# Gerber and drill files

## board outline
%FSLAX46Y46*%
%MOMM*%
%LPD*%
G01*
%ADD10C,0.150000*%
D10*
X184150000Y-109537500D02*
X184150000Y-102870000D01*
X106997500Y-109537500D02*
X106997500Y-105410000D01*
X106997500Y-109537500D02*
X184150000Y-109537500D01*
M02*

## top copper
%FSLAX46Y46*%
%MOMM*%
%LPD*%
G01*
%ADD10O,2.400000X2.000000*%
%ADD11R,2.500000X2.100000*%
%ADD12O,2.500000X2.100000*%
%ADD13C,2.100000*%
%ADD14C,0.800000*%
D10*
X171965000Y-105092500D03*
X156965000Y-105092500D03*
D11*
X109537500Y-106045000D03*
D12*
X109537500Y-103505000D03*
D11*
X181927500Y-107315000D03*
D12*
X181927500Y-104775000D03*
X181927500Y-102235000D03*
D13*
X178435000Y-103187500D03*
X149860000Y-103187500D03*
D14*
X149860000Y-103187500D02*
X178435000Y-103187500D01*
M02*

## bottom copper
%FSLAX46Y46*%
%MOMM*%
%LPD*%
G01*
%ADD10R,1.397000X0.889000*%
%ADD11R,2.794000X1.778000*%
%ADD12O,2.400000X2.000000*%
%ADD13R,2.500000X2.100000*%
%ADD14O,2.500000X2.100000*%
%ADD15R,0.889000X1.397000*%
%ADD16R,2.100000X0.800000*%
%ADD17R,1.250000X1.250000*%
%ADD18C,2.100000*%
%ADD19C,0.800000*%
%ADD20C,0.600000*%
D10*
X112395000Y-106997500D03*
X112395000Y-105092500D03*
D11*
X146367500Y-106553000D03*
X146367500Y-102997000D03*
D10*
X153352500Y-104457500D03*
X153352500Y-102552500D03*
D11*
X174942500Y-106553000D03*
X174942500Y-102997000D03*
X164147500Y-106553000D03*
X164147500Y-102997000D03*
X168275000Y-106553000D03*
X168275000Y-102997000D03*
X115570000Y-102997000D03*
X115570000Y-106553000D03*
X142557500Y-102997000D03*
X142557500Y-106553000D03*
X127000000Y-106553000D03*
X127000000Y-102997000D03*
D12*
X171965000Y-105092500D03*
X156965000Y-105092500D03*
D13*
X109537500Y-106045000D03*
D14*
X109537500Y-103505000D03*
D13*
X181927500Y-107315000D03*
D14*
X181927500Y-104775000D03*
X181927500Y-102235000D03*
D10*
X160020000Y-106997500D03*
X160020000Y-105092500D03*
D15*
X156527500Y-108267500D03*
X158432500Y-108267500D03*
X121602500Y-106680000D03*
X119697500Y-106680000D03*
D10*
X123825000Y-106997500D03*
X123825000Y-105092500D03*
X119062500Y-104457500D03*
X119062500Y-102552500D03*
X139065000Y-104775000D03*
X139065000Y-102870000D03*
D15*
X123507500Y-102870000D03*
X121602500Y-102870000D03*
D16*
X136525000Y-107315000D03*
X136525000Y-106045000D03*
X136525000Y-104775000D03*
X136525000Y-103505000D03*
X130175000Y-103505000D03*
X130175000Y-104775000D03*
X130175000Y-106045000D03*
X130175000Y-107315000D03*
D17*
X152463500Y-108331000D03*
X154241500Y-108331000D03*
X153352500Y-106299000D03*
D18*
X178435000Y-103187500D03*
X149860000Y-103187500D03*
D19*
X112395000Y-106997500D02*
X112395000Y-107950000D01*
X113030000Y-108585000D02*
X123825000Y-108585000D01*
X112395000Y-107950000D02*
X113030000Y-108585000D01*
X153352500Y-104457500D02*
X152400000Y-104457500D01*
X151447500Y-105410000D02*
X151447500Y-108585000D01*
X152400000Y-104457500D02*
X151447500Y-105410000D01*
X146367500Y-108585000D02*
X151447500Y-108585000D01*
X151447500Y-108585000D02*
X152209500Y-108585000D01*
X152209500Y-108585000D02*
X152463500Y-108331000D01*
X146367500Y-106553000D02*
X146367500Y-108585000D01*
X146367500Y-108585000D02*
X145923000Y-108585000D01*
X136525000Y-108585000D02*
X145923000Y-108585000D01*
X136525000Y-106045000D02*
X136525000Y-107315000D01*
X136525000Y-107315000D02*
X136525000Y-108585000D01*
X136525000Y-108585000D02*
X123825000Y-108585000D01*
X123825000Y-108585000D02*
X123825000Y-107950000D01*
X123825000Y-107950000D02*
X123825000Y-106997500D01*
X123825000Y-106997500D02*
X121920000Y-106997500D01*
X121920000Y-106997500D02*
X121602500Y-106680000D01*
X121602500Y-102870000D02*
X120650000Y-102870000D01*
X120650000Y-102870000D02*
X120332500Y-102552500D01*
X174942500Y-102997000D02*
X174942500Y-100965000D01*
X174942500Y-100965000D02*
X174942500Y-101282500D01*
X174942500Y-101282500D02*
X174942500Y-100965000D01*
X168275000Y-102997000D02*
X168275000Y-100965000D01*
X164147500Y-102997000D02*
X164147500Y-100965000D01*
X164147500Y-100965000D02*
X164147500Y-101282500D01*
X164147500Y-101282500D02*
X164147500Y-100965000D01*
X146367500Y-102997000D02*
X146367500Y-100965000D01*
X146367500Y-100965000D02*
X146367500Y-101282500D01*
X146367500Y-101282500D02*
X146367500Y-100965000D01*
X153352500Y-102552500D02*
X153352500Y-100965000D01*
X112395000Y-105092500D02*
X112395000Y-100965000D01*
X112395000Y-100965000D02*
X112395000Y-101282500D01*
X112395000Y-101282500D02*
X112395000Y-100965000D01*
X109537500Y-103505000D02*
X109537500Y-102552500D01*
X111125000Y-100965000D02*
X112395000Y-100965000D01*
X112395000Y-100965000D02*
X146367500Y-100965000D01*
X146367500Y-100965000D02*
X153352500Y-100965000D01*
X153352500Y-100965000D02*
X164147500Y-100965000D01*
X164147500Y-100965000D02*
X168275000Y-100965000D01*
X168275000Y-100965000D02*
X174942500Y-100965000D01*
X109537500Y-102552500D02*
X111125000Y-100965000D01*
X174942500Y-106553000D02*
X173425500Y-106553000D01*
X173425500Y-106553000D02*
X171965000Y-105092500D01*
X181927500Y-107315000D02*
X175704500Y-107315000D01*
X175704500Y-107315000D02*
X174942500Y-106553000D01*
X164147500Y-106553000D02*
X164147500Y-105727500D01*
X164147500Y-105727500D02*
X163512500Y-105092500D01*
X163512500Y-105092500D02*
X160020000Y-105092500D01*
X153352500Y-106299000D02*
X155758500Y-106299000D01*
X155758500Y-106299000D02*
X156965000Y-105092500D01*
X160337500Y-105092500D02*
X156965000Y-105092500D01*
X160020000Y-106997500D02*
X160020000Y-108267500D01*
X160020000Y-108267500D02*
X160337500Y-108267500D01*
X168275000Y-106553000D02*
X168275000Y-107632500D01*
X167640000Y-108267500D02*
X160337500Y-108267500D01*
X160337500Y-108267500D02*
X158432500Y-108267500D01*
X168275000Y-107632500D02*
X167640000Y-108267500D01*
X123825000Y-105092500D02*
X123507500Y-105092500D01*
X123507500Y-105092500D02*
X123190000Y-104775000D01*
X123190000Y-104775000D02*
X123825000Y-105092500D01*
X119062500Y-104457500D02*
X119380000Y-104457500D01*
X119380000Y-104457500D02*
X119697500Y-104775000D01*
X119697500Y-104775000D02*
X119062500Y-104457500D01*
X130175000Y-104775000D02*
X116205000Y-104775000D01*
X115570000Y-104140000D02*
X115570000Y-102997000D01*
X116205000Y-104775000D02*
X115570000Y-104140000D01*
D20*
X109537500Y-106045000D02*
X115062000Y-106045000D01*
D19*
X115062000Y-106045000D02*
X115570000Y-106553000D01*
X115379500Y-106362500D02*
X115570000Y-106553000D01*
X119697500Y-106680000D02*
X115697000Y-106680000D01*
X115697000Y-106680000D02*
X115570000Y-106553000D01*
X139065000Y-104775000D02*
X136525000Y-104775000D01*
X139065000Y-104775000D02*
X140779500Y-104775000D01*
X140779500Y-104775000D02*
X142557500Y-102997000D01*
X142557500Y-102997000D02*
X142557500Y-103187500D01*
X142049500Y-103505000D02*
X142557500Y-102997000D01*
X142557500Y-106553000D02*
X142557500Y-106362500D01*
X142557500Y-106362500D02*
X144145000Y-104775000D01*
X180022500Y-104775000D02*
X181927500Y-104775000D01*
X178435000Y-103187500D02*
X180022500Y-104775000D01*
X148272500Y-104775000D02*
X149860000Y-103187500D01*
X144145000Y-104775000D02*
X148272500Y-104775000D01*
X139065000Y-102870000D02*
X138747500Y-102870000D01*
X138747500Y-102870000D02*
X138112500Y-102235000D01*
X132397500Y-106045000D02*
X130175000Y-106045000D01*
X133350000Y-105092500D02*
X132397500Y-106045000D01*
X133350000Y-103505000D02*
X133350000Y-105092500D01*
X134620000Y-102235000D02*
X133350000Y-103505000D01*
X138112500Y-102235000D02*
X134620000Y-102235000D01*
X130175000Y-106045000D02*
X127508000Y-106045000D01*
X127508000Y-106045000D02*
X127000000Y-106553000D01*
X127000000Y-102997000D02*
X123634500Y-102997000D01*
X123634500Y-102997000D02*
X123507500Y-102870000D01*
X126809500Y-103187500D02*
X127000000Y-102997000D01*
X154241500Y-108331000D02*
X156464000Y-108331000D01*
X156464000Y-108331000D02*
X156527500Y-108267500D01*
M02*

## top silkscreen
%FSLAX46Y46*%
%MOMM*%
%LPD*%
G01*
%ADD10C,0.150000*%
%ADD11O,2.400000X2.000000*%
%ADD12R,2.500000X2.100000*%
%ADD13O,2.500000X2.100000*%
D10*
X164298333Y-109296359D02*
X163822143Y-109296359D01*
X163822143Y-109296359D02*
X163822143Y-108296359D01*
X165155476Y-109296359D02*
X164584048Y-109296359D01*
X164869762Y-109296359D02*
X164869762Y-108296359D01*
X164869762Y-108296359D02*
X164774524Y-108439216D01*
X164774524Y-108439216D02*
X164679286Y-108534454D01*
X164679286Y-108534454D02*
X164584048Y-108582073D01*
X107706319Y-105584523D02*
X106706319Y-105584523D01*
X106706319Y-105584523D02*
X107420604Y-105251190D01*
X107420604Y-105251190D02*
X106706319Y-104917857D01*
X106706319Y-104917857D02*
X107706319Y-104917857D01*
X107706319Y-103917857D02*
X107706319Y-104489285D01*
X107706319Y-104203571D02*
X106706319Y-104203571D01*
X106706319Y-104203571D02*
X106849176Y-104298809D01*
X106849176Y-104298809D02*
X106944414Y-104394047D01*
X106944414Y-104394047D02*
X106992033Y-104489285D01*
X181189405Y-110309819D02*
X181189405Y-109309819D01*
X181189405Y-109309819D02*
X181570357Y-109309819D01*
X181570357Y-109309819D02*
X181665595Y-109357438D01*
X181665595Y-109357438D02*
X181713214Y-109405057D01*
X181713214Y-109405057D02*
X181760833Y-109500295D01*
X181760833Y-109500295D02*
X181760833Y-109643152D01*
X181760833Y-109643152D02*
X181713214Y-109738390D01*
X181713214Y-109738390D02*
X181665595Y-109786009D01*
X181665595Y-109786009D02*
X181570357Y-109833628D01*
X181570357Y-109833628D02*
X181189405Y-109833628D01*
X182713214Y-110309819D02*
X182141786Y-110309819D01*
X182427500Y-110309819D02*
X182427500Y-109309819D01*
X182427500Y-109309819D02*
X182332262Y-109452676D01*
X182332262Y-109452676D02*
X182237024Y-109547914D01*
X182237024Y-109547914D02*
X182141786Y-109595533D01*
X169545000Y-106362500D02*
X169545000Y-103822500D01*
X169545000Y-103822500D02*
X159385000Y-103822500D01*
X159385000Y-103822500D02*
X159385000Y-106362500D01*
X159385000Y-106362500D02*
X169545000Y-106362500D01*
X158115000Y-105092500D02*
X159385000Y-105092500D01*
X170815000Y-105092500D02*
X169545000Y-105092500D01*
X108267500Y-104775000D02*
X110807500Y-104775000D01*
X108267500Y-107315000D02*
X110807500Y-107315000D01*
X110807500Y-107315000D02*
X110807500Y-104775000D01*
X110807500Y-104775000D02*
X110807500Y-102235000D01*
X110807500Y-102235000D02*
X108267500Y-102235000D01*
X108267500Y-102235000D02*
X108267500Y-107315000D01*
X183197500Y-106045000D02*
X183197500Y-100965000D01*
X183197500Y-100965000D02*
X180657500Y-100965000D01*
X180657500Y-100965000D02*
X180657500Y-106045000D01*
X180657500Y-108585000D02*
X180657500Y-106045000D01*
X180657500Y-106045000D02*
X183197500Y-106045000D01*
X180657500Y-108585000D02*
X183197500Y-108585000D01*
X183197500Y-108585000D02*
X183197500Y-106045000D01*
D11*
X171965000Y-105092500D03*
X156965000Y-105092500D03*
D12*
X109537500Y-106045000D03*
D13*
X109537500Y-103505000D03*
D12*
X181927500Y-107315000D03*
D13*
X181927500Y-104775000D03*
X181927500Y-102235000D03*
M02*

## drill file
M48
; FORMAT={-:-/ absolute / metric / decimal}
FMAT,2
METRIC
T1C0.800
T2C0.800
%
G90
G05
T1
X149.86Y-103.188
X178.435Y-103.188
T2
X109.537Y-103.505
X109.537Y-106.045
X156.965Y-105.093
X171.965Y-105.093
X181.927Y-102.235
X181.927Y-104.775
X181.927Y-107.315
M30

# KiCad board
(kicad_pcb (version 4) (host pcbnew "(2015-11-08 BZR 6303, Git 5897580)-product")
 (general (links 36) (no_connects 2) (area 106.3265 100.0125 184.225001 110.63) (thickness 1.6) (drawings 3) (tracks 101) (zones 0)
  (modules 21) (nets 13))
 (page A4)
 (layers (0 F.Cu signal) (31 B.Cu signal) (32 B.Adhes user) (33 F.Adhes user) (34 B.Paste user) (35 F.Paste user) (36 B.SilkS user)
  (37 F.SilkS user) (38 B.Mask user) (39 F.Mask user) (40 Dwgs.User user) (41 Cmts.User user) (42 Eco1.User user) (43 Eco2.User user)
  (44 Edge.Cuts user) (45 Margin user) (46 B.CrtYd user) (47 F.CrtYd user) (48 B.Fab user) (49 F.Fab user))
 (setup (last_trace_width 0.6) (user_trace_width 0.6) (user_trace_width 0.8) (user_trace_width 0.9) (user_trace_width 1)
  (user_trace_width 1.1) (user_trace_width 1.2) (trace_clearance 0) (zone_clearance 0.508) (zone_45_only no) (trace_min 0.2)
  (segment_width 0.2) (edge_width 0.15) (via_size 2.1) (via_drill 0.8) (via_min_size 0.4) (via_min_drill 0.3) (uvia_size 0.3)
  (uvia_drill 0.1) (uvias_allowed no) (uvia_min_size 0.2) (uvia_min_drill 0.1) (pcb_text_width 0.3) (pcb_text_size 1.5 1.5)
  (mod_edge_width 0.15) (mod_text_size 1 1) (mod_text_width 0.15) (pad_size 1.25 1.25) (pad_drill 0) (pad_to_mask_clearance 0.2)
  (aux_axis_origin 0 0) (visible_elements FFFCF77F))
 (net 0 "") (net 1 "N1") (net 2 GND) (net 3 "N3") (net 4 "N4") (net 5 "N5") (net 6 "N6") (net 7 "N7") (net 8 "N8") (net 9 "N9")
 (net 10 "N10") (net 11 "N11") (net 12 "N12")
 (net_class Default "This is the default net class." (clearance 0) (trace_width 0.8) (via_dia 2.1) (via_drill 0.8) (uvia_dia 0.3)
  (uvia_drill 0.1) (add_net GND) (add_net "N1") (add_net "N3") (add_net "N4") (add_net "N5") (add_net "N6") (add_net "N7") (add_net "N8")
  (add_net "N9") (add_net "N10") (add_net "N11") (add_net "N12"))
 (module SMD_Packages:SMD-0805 (layer B.Cu) (at 112.395 106.045 90)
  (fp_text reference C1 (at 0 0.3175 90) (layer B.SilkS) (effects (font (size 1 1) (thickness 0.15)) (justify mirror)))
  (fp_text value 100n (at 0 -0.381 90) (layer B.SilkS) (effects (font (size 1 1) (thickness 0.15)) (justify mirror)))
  (pad 1 smd rect (at -0.9525 0 90) (size 0.889 1.397) (layers B.Cu B.Paste B.Mask) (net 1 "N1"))
  (pad 2 smd rect (at 0.9525 0 90) (size 0.889 1.397) (layers B.Cu B.Paste B.Mask) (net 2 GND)))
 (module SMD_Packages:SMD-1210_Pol (layer B.Cu) (at 146.3675 104.775 90)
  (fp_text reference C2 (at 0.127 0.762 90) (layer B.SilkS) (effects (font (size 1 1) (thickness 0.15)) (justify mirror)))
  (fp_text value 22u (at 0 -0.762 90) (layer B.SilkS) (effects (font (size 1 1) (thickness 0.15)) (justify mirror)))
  (pad 1 smd rect (at -1.778 0 90) (size 1.778 2.794) (layers B.Cu B.Paste B.Mask) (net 1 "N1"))
  (pad 2 smd rect (at 1.778 0 90) (size 1.778 2.794) (layers B.Cu B.Paste B.Mask) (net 2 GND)))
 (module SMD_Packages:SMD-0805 (layer B.Cu) (at 153.3525 103.505 90)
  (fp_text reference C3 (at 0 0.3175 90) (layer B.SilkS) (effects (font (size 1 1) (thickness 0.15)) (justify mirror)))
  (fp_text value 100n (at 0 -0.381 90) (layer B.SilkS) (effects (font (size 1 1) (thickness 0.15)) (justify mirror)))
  (pad 1 smd rect (at -0.9525 0 90) (size 0.889 1.397) (layers B.Cu B.Paste B.Mask) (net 1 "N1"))
  (pad 2 smd rect (at 0.9525 0 90) (size 0.889 1.397) (layers B.Cu B.Paste B.Mask) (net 2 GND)))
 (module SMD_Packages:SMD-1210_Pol (layer B.Cu) (at 174.9425 104.775 90)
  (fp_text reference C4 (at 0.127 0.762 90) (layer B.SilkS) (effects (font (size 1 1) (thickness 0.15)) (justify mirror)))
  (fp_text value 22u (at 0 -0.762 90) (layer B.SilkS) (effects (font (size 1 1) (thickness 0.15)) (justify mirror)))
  (pad 1 smd rect (at -1.778 0 90) (size 1.778 2.794) (layers B.Cu B.Paste B.Mask) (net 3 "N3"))
  (pad 2 smd rect (at 1.778 0 90) (size 1.778 2.794) (layers B.Cu B.Paste B.Mask) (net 2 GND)))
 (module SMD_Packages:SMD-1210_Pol (layer B.Cu) (at 164.1475 104.775 90)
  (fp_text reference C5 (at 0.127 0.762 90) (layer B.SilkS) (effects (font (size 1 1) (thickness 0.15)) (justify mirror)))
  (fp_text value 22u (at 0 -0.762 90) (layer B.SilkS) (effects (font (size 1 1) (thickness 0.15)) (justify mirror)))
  (pad 1 smd rect (at -1.778 0 90) (size 1.778 2.794) (layers B.Cu B.Paste B.Mask) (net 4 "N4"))
  (pad 2 smd rect (at 1.778 0 90) (size 1.778 2.794) (layers B.Cu B.Paste B.Mask) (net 2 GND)))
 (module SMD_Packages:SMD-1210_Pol (layer B.Cu) (at 168.275 104.775 90)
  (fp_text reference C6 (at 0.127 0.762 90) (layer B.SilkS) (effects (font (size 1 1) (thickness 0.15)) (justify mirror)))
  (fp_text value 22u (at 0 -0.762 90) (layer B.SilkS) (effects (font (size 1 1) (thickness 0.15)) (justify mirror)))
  (pad 1 smd rect (at -1.778 0 90) (size 1.778 2.794) (layers B.Cu B.Paste B.Mask) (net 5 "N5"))
  (pad 2 smd rect (at 1.778 0 90) (size 1.778 2.794) (layers B.Cu B.Paste B.Mask) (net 2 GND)))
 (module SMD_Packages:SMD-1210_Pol (layer B.Cu) (at 115.57 104.775 270)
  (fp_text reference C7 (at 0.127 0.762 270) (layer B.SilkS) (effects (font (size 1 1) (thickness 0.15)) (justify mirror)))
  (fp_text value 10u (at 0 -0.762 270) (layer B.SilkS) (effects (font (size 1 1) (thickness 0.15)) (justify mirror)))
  (pad 1 smd rect (at -1.778 0 270) (size 1.778 2.794) (layers B.Cu B.Paste B.Mask) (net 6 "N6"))
  (pad 2 smd rect (at 1.778 0 270) (size 1.778 2.794) (layers B.Cu B.Paste B.Mask) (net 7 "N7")))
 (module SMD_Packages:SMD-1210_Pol (layer B.Cu) (at 142.5575 104.775 270)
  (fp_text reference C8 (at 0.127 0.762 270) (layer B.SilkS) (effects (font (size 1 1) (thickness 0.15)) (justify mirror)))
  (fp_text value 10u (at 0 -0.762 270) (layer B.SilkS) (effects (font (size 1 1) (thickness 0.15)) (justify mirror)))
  (pad 1 smd rect (at -1.778 0 270) (size 1.778 2.794) (layers B.Cu B.Paste B.Mask) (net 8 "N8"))
  (pad 2 smd rect (at 1.778 0 270) (size 1.778 2.794) (layers B.Cu B.Paste B.Mask) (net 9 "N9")))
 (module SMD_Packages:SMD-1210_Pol (layer B.Cu) (at 127 104.775 90)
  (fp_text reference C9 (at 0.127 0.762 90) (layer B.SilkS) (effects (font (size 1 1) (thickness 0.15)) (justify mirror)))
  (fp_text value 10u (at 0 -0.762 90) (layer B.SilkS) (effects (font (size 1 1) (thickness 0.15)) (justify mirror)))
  (pad 1 smd rect (at -1.778 0 90) (size 1.778 2.794) (layers B.Cu B.Paste B.Mask) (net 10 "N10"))
  (pad 2 smd rect (at 1.778 0 90) (size 1.778 2.794) (layers B.Cu B.Paste B.Mask) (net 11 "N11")))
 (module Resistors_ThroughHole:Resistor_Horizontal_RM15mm (layer F.Cu) (at 164.465 105.0925 180)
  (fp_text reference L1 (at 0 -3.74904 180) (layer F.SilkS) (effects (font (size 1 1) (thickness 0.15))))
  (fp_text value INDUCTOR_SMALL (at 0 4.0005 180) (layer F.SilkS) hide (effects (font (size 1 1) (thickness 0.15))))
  (fp_line (start -5.08 -1.27) (end -5.08 1.27) (layer F.SilkS) (width 0.15))
  (fp_line (start -5.08 1.27) (end 5.08 1.27) (layer F.SilkS) (width 0.15))
  (fp_line (start 5.08 1.27) (end 5.08 -1.27) (layer F.SilkS) (width 0.15))
  (fp_line (start 5.08 -1.27) (end -5.08 -1.27) (layer F.SilkS) (width 0.15))
  (fp_line (start 6.35 0) (end 5.08 0) (layer F.SilkS) (width 0.15))
  (fp_line (start -6.35 0) (end -5.08 0) (layer F.SilkS) (width 0.15))
  (pad 1 thru_hole oval (at -7.5 0 180) (size 2.4 2) (drill 0.8) (layers *.Cu *.SilkS *.Mask) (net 3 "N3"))
  (pad 2 thru_hole oval (at 7.5 0 180) (size 2.4 2) (drill 0.8) (layers *.Cu *.SilkS *.Mask) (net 4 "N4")))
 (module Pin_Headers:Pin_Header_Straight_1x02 (layer F.Cu) (at 109.5375 104.775 90)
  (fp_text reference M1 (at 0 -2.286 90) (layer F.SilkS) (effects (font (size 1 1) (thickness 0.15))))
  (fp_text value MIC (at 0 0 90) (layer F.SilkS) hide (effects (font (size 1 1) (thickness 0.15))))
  (fp_line (start 0 -1.27) (end 0 1.27) (layer F.SilkS) (width 0.15))
  (fp_line (start -2.54 -1.27) (end -2.54 1.27) (layer F.SilkS) (width 0.15))
  (fp_line (start -2.54 1.27) (end 0 1.27) (layer F.SilkS) (width 0.15))
  (fp_line (start 0 1.27) (end 2.54 1.27) (layer F.SilkS) (width 0.15))
  (fp_line (start 2.54 1.27) (end 2.54 -1.27) (layer F.SilkS) (width 0.15))
  (fp_line (start 2.54 -1.27) (end -2.54 -1.27) (layer F.SilkS) (width 0.15))
  (pad 1 thru_hole rect (at -1.27 0 90) (size 2.1 2.5) (drill 0.8) (layers *.Cu *.Mask F.SilkS) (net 7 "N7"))
  (pad 2 thru_hole oval (at 1.27 0 90) (size 2.1 2.5) (drill 0.8) (layers *.Cu *.Mask F.SilkS) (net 2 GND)))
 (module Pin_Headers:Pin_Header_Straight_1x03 (layer F.Cu) (at 181.9275 104.775 90)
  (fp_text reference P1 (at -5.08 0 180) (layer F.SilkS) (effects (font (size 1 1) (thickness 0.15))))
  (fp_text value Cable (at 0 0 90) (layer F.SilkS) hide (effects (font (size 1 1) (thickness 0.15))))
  (fp_line (start -1.27 1.27) (end 3.81 1.27) (layer F.SilkS) (width 0.15))
  (fp_line (start 3.81 1.27) (end 3.81 -1.27) (layer F.SilkS) (width 0.15))
  (fp_line (start 3.81 -1.27) (end -1.27 -1.27) (layer F.SilkS) (width 0.15))
  (fp_line (start -3.81 -1.27) (end -1.27 -1.27) (layer F.SilkS) (width 0.15))
  (fp_line (start -1.27 -1.27) (end -1.27 1.27) (layer F.SilkS) (width 0.15))
  (fp_line (start -3.81 -1.27) (end -3.81 1.27) (layer F.SilkS) (width 0.15))
  (fp_line (start -3.81 1.27) (end -1.27 1.27) (layer F.SilkS) (width 0.15))
  (pad 1 thru_hole rect (at -2.54 0 90) (size 2.1 2.5) (drill 0.8) (layers *.Cu *.Mask F.SilkS) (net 3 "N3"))
  (pad 2 thru_hole oval (at 0 0 90) (size 2.1 2.5) (drill 0.8) (layers *.Cu *.Mask F.SilkS) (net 9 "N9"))
  (pad 3 thru_hole oval (at 2.54 0 90) (size 2.1 2.5) (drill 0.8) (layers *.Cu *.Mask F.SilkS) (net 2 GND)))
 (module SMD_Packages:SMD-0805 (layer B.Cu) (at 160.02 106.045 90)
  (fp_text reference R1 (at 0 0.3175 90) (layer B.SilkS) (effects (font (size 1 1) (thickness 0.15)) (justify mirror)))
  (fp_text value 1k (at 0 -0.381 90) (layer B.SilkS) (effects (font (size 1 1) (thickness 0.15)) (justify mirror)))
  (pad 1 smd rect (at -0.9525 0 90) (size 0.889 1.397) (layers B.Cu B.Paste B.Mask) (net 5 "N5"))
  (pad 2 smd rect (at 0.9525 0 90) (size 0.889 1.397) (layers B.Cu B.Paste B.Mask) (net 4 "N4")))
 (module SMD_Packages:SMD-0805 (layer B.Cu) (at 157.48 108.2675)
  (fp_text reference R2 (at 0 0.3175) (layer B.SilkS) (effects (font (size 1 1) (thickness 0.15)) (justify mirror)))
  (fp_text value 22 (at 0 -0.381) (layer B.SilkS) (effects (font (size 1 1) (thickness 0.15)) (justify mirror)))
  (pad 1 smd rect (at -0.9525 0) (size 0.889 1.397) (layers B.Cu B.Paste B.Mask) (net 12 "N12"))
  (pad 2 smd rect (at 0.9525 0) (size 0.889 1.397) (layers B.Cu B.Paste B.Mask) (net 5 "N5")))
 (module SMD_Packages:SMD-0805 (layer B.Cu) (at 120.65 106.68 180)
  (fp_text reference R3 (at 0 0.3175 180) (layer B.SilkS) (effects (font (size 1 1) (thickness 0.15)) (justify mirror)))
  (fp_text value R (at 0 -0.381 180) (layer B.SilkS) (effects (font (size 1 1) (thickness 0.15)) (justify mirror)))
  (pad 1 smd rect (at -0.9525 0 180) (size 0.889 1.397) (layers B.Cu B.Paste B.Mask) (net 1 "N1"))
  (pad 2 smd rect (at 0.9525 0 180) (size 0.889 1.397) (layers B.Cu B.Paste B.Mask) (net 7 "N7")))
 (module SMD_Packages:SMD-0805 (layer B.Cu) (at 123.825 106.045 90)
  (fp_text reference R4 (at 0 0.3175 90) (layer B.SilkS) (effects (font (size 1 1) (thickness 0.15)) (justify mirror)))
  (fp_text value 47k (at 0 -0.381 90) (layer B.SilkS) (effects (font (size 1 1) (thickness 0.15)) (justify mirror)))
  (pad 1 smd rect (at -0.9525 0 90) (size 0.889 1.397) (layers B.Cu B.Paste B.Mask) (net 1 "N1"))
  (pad 2 smd rect (at 0.9525 0 90) (size 0.889 1.397) (layers B.Cu B.Paste B.Mask) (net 6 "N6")))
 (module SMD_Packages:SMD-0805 (layer B.Cu) (at 119.0625 103.505 90)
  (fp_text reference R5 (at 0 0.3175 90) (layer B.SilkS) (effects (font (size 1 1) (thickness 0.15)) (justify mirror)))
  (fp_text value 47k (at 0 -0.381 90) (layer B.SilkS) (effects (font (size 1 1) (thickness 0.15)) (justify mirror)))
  (pad 1 smd rect (at -0.9525 0 90) (size 0.889 1.397) (layers B.Cu B.Paste B.Mask) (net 6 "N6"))
  (pad 2 smd rect (at 0.9525 0 90) (size 0.889 1.397) (layers B.Cu B.Paste B.Mask) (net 2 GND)))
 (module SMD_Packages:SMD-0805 (layer B.Cu) (at 139.065 103.8225 90)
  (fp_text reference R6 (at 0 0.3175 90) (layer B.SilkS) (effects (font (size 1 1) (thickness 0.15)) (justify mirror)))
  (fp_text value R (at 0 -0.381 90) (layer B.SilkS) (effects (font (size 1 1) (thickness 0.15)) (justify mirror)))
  (pad 1 smd rect (at -0.9525 0 90) (size 0.889 1.397) (layers B.Cu B.Paste B.Mask) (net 8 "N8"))
  (pad 2 smd rect (at 0.9525 0 90) (size 0.889 1.397) (layers B.Cu B.Paste B.Mask) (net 10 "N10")))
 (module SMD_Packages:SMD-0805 (layer B.Cu) (at 122.555 102.87 180)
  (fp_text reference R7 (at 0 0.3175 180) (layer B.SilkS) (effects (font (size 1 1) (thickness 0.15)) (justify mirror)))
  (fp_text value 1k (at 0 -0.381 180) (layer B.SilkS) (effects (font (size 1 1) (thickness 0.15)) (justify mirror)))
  (pad 1 smd rect (at -0.9525 0 180) (size 0.889 1.397) (layers B.Cu B.Paste B.Mask) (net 11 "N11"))
  (pad 2 smd rect (at 0.9525 0 180) (size 0.889 1.397) (layers B.Cu B.Paste B.Mask) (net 2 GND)))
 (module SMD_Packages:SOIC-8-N (layer B.Cu) (at 133.35 105.41 90)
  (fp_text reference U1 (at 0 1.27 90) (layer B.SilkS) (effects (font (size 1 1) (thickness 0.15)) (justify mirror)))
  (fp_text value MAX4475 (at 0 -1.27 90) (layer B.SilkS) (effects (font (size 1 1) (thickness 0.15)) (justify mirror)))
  (pad 8 smd rect (at -1.905 3.175 90) (size 0.8 2.1) (layers B.Cu B.Paste B.Mask) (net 1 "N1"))
  (pad 7 smd rect (at -0.635 3.175 90) (size 0.8 2.1) (layers B.Cu B.Paste B.Mask) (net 1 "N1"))
  (pad 6 smd rect (at 0.635 3.175 90) (size 0.8 2.1) (layers B.Cu B.Paste B.Mask) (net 8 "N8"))
  (pad 5 smd rect (at 1.905 3.175 90) (size 0.8 2.1) (layers B.Cu B.Paste B.Mask))
  (pad 4 smd rect (at 1.905 -3.175 90) (size 0.8 2.1) (layers B.Cu B.Paste B.Mask) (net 2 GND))
  (pad 3 smd rect (at 0.635 -3.175 90) (size 0.8 2.1) (layers B.Cu B.Paste B.Mask) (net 6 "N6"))
  (pad 2 smd rect (at -0.635 -3.175 90) (size 0.8 2.1) (layers B.Cu B.Paste B.Mask) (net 10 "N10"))
  (pad 1 smd rect (at -1.905 -3.175 90) (size 0.8 2.1) (layers B.Cu B.Paste B.Mask)))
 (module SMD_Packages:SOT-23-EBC (layer B.Cu) (at 153.3525 107.315)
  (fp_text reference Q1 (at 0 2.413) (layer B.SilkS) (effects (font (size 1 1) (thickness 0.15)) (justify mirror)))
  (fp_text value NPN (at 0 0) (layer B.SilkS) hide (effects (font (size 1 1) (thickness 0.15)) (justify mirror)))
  (pad 1 smd rect (at -0.889 1.016) (size 1.25 1.25) (layers B.Cu B.Paste B.Mask) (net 1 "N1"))
  (pad 2 smd rect (at 0.889 1.016) (size 1.25 1.25) (layers B.Cu B.Paste B.Mask) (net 12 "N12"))
  (pad 3 smd rect (at 0 -1.016) (size 1.25 1.25) (layers B.Cu B.Paste B.Mask) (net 4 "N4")))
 (gr_line (start 184.15 109.5375) (end 184.15 102.87) (angle 90) (layer Edge.Cuts) (width 0.15))
 (gr_line (start 106.9975 109.5375) (end 106.9975 105.41) (angle 90) (layer Edge.Cuts) (width 0.15))
 (gr_line (start 106.9975 109.5375) (end 184.15 109.5375) (angle 90) (layer Edge.Cuts) (width 0.15))
 (segment (start 112.395 106.9975) (end 112.395 107.95) (width 0.8) (layer B.Cu) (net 1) (status 400000))
 (segment (start 113.03 108.585) (end 123.825 108.585) (width 0.8) (layer B.Cu) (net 1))
 (segment (start 112.395 107.95) (end 113.03 108.585) (width 0.8) (layer B.Cu) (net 1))
 (segment (start 153.3525 104.4575) (end 152.4 104.4575) (width 0.8) (layer B.Cu) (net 1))
 (segment (start 151.4475 105.41) (end 151.4475 108.585) (width 0.8) (layer B.Cu) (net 1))
 (segment (start 152.4 104.4575) (end 151.4475 105.41) (width 0.8) (layer B.Cu) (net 1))
 (segment (start 146.3675 108.585) (end 151.4475 108.585) (width 0.8) (layer B.Cu) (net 1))
 (segment (start 151.4475 108.585) (end 152.2095 108.585) (width 0.8) (layer B.Cu) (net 1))
 (segment (start 152.2095 108.585) (end 152.4635 108.331) (width 0.8) (layer B.Cu) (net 1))
 (segment (start 146.3675 106.553) (end 146.3675 108.585) (width 0.8) (layer B.Cu) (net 1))
 (segment (start 146.3675 108.585) (end 145.923 108.585) (width 0.8) (layer B.Cu) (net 1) (status 20))
 (segment (start 136.525 108.585) (end 145.923 108.585) (width 0.8) (layer B.Cu) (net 1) (status 20))
 (segment (start 136.525 106.045) (end 136.525 107.315) (width 0.8) (layer B.Cu) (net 1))
 (segment (start 136.525 107.315) (end 136.525 108.585) (width 0.8) (layer B.Cu) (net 1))
 (segment (start 136.525 108.585) (end 123.825 108.585) (width 0.8) (layer B.Cu) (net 1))
 (segment (start 123.825 108.585) (end 123.825 107.95) (width 0.8) (layer B.Cu) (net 1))
 (segment (start 123.825 107.95) (end 123.825 106.9975) (width 0.8) (layer B.Cu) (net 1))
 (segment (start 123.825 106.9975) (end 121.92 106.9975) (width 0.8) (layer B.Cu) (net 1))
 (segment (start 121.92 106.9975) (end 121.6025 106.68) (width 0.8) (layer B.Cu) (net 1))
 (segment (start 121.6025 102.87) (end 120.65 102.87) (width 0.8) (layer B.Cu) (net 2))
 (segment (start 120.65 102.87) (end 120.3325 102.5525) (width 0.8) (layer B.Cu) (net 2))
 (segment (start 174.9425 102.997) (end 174.9425 100.965) (width 0.8) (layer B.Cu) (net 2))
 (segment (start 174.9425 100.965) (end 174.9425 101.2825) (width 0.8) (layer B.Cu) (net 2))
 (segment (start 174.9425 101.2825) (end 174.9425 100.965) (width 0.8) (layer B.Cu) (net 2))
 (segment (start 168.275 102.997) (end 168.275 100.965) (width 0.8) (layer B.Cu) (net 2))
 (segment (start 164.1475 102.997) (end 164.1475 100.965) (width 0.8) (layer B.Cu) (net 2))
 (segment (start 164.1475 100.965) (end 164.1475 101.2825) (width 0.8) (layer B.Cu) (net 2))
 (segment (start 164.1475 101.2825) (end 164.1475 100.965) (width 0.8) (layer B.Cu) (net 2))
 (segment (start 146.3675 102.997) (end 146.3675 100.965) (width 0.8) (layer B.Cu) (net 2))
 (segment (start 146.3675 100.965) (end 146.3675 101.2825) (width 0.8) (layer B.Cu) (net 2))
 (segment (start 146.3675 101.2825) (end 146.3675 100.965) (width 0.8) (layer B.Cu) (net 2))
 (segment (start 153.3525 102.5525) (end 153.3525 100.965) (width 0.8) (layer B.Cu) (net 2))
 (segment (start 112.395 105.0925) (end 112.395 100.965) (width 0.8) (layer B.Cu) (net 2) (status 10))
 (segment (start 112.395 100.965) (end 112.395 101.2825) (width 0.8) (layer B.Cu) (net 2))
 (segment (start 112.395 101.2825) (end 112.395 100.965) (width 0.8) (layer B.Cu) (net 2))
 (segment (start 109.5375 103.505) (end 109.5375 102.5525) (width 0.8) (layer B.Cu) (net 2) (status 10))
 (segment (start 111.125 100.965) (end 112.395 100.965) (width 0.8) (layer B.Cu) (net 2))
 (segment (start 112.395 100.965) (end 146.3675 100.965) (width 0.8) (layer B.Cu) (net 2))
 (segment (start 146.3675 100.965) (end 153.3525 100.965) (width 0.8) (layer B.Cu) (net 2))
 (segment (start 153.3525 100.965) (end 164.1475 100.965) (width 0.8) (layer B.Cu) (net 2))
 (segment (start 164.1475 100.965) (end 168.275 100.965) (width 0.8) (layer B.Cu) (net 2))
 (segment (start 168.275 100.965) (end 174.9425 100.965) (width 0.8) (layer B.Cu) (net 2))
 (segment (start 109.5375 102.5525) (end 111.125 100.965) (width 0.8) (layer B.Cu) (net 2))
 (segment (start 174.9425 106.553) (end 173.4255 106.553) (width 0.8) (layer B.Cu) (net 3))
 (segment (start 173.4255 106.553) (end 171.965 105.0925) (width 0.8) (layer B.Cu) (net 3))
 (segment (start 181.9275 107.315) (end 175.7045 107.315) (width 0.8) (layer B.Cu) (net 3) (status 10))
 (segment (start 175.7045 107.315) (end 174.9425 106.553) (width 0.8) (layer B.Cu) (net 3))
 (segment (start 164.1475 106.553) (end 164.1475 105.7275) (width 0.8) (layer B.Cu) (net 4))
 (segment (start 164.1475 105.7275) (end 163.5125 105.0925) (width 0.8) (layer B.Cu) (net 4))
 (segment (start 163.5125 105.0925) (end 160.02 105.0925) (width 0.8) (layer B.Cu) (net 4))
 (segment (start 153.3525 106.299) (end 155.7585 106.299) (width 0.8) (layer B.Cu) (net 4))
 (segment (start 155.7585 106.299) (end 156.965 105.0925) (width 0.8) (layer B.Cu) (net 4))
 (segment (start 160.3375 105.0925) (end 156.965 105.0925) (width 0.8) (layer B.Cu) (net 4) (status 20))
 (segment (start 160.02 106.9975) (end 160.02 108.2675) (width 0.8) (layer B.Cu) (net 5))
 (segment (start 160.02 108.2675) (end 160.3375 108.2675) (width 0.8) (layer B.Cu) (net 5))
 (segment (start 168.275 106.553) (end 168.275 107.6325) (width 0.8) (layer B.Cu) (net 5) (status 10))
 (segment (start 167.64 108.2675) (end 160.3375 108.2675) (width 0.8) (layer B.Cu) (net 5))
 (segment (start 160.3375 108.2675) (end 158.4325 108.2675) (width 0.8) (layer B.Cu) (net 5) (status 20))
 (segment (start 168.275 107.6325) (end 167.64 108.2675) (width 0.8) (layer B.Cu) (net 5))
 (segment (start 123.825 105.0925) (end 123.5075 105.0925) (width 0.8) (layer B.Cu) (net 6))
 (segment (start 123.5075 105.0925) (end 123.19 104.775) (width 0.8) (layer B.Cu) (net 6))
 (segment (start 123.19 104.775) (end 123.825 105.0925) (width 0.8) (layer B.Cu) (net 6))
 (segment (start 119.0625 104.4575) (end 119.38 104.4575) (width 0.8) (layer B.Cu) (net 6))
 (segment (start 119.38 104.4575) (end 119.6975 104.775) (width 0.8) (layer B.Cu) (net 6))
 (segment (start 119.6975 104.775) (end 119.0625 104.4575) (width 0.8) (layer B.Cu) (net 6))
 (segment (start 130.175 104.775) (end 116.205 104.775) (width 0.8) (layer B.Cu) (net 6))
 (segment (start 115.57 104.14) (end 115.57 102.997) (width 0.8) (layer B.Cu) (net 6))
 (segment (start 116.205 104.775) (end 115.57 104.14) (width 0.8) (layer B.Cu) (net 6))
 (segment (start 109.5375 106.045) (end 115.062 106.045) (width 0.6) (layer B.Cu) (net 7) (status C00000))
 (segment (start 115.062 106.045) (end 115.57 106.553) (width 0.8) (layer B.Cu) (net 7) (status C00000))
 (segment (start 115.3795 106.3625) (end 115.57 106.553) (width 0.8) (layer B.Cu) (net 7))
 (segment (start 119.6975 106.68) (end 115.697 106.68) (width 0.8) (layer B.Cu) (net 7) (status 20))
 (segment (start 115.697 106.68) (end 115.57 106.553) (width 0.8) (layer B.Cu) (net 7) (status 30))
 (segment (start 139.065 104.775) (end 136.525 104.775) (width 0.8) (layer B.Cu) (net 8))
 (segment (start 139.065 104.775) (end 140.7795 104.775) (width 0.8) (layer B.Cu) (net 8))
 (segment (start 140.7795 104.775) (end 142.5575 102.997) (width 0.8) (layer B.Cu) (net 8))
 (segment (start 142.5575 102.997) (end 142.5575 103.1875) (width 0.8) (layer B.Cu) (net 8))
 (segment (start 142.0495 103.505) (end 142.5575 102.997) (width 0.8) (layer B.Cu) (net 8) (status 30))
 (segment (start 142.5575 106.553) (end 142.5575 106.3625) (width 0.8) (layer B.Cu) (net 9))
 (segment (start 142.5575 106.3625) (end 144.145 104.775) (width 0.8) (layer B.Cu) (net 9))
 (segment (start 180.0225 104.775) (end 181.9275 104.775) (width 0.8) (layer B.Cu) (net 9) (status 20))
 (segment (start 178.435 103.1875) (end 180.0225 104.775) (width 0.8) (layer B.Cu) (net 9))
 (via (at 178.435 103.1875) (size 2.1) (drill 0.8) (layers F.Cu B.Cu) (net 9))
 (segment (start 149.86 103.1875) (end 178.435 103.1875) (width 0.8) (layer F.Cu) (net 9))
 (via (at 149.86 103.1875) (size 2.1) (drill 0.8) (layers F.Cu B.Cu) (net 9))
 (segment (start 148.2725 104.775) (end 149.86 103.1875) (width 0.8) (layer B.Cu) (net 9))
 (segment (start 144.145 104.775) (end 148.2725 104.775) (width 0.8) (layer B.Cu) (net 9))
 (segment (start 139.065 102.87) (end 138.7475 102.87) (width 0.8) (layer B.Cu) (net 10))
 (segment (start 138.7475 102.87) (end 138.1125 102.235) (width 0.8) (layer B.Cu) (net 10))
 (segment (start 132.3975 106.045) (end 130.175 106.045) (width 0.8) (layer B.Cu) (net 10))
 (segment (start 133.35 105.0925) (end 132.3975 106.045) (width 0.8) (layer B.Cu) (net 10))
 (segment (start 133.35 103.505) (end 133.35 105.0925) (width 0.8) (layer B.Cu) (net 10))
 (segment (start 134.62 102.235) (end 133.35 103.505) (width 0.8) (layer B.Cu) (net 10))
 (segment (start 138.1125 102.235) (end 134.62 102.235) (width 0.8) (layer B.Cu) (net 10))
 (segment (start 130.175 106.045) (end 127.508 106.045) (width 0.8) (layer B.Cu) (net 10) (status 10))
 (segment (start 127.508 106.045) (end 127 106.553) (width 0.8) (layer B.Cu) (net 10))
 (segment (start 127 102.997) (end 123.6345 102.997) (width 0.8) (layer B.Cu) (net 11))
 (segment (start 123.6345 102.997) (end 123.5075 102.87) (width 0.8) (layer B.Cu) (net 11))
 (segment (start 126.8095 103.1875) (end 127 102.997) (width 0.8) (layer B.Cu) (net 11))
 (segment (start 154.2415 108.331) (end 156.464 108.331) (width 0.8) (layer B.Cu) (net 12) (status 20))
 (segment (start 156.464 108.331) (end 156.5275 108.2675) (width 0.8) (layer B.Cu) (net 12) (status 30))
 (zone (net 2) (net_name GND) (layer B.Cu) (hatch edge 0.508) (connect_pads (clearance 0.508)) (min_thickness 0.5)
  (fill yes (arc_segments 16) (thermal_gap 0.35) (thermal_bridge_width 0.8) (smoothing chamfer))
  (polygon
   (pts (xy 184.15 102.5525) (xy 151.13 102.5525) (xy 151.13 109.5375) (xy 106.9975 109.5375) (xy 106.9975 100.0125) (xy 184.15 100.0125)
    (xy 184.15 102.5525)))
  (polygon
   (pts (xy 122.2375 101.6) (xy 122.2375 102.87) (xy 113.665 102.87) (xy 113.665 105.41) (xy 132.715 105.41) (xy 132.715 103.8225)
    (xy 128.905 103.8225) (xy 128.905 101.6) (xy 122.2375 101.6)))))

